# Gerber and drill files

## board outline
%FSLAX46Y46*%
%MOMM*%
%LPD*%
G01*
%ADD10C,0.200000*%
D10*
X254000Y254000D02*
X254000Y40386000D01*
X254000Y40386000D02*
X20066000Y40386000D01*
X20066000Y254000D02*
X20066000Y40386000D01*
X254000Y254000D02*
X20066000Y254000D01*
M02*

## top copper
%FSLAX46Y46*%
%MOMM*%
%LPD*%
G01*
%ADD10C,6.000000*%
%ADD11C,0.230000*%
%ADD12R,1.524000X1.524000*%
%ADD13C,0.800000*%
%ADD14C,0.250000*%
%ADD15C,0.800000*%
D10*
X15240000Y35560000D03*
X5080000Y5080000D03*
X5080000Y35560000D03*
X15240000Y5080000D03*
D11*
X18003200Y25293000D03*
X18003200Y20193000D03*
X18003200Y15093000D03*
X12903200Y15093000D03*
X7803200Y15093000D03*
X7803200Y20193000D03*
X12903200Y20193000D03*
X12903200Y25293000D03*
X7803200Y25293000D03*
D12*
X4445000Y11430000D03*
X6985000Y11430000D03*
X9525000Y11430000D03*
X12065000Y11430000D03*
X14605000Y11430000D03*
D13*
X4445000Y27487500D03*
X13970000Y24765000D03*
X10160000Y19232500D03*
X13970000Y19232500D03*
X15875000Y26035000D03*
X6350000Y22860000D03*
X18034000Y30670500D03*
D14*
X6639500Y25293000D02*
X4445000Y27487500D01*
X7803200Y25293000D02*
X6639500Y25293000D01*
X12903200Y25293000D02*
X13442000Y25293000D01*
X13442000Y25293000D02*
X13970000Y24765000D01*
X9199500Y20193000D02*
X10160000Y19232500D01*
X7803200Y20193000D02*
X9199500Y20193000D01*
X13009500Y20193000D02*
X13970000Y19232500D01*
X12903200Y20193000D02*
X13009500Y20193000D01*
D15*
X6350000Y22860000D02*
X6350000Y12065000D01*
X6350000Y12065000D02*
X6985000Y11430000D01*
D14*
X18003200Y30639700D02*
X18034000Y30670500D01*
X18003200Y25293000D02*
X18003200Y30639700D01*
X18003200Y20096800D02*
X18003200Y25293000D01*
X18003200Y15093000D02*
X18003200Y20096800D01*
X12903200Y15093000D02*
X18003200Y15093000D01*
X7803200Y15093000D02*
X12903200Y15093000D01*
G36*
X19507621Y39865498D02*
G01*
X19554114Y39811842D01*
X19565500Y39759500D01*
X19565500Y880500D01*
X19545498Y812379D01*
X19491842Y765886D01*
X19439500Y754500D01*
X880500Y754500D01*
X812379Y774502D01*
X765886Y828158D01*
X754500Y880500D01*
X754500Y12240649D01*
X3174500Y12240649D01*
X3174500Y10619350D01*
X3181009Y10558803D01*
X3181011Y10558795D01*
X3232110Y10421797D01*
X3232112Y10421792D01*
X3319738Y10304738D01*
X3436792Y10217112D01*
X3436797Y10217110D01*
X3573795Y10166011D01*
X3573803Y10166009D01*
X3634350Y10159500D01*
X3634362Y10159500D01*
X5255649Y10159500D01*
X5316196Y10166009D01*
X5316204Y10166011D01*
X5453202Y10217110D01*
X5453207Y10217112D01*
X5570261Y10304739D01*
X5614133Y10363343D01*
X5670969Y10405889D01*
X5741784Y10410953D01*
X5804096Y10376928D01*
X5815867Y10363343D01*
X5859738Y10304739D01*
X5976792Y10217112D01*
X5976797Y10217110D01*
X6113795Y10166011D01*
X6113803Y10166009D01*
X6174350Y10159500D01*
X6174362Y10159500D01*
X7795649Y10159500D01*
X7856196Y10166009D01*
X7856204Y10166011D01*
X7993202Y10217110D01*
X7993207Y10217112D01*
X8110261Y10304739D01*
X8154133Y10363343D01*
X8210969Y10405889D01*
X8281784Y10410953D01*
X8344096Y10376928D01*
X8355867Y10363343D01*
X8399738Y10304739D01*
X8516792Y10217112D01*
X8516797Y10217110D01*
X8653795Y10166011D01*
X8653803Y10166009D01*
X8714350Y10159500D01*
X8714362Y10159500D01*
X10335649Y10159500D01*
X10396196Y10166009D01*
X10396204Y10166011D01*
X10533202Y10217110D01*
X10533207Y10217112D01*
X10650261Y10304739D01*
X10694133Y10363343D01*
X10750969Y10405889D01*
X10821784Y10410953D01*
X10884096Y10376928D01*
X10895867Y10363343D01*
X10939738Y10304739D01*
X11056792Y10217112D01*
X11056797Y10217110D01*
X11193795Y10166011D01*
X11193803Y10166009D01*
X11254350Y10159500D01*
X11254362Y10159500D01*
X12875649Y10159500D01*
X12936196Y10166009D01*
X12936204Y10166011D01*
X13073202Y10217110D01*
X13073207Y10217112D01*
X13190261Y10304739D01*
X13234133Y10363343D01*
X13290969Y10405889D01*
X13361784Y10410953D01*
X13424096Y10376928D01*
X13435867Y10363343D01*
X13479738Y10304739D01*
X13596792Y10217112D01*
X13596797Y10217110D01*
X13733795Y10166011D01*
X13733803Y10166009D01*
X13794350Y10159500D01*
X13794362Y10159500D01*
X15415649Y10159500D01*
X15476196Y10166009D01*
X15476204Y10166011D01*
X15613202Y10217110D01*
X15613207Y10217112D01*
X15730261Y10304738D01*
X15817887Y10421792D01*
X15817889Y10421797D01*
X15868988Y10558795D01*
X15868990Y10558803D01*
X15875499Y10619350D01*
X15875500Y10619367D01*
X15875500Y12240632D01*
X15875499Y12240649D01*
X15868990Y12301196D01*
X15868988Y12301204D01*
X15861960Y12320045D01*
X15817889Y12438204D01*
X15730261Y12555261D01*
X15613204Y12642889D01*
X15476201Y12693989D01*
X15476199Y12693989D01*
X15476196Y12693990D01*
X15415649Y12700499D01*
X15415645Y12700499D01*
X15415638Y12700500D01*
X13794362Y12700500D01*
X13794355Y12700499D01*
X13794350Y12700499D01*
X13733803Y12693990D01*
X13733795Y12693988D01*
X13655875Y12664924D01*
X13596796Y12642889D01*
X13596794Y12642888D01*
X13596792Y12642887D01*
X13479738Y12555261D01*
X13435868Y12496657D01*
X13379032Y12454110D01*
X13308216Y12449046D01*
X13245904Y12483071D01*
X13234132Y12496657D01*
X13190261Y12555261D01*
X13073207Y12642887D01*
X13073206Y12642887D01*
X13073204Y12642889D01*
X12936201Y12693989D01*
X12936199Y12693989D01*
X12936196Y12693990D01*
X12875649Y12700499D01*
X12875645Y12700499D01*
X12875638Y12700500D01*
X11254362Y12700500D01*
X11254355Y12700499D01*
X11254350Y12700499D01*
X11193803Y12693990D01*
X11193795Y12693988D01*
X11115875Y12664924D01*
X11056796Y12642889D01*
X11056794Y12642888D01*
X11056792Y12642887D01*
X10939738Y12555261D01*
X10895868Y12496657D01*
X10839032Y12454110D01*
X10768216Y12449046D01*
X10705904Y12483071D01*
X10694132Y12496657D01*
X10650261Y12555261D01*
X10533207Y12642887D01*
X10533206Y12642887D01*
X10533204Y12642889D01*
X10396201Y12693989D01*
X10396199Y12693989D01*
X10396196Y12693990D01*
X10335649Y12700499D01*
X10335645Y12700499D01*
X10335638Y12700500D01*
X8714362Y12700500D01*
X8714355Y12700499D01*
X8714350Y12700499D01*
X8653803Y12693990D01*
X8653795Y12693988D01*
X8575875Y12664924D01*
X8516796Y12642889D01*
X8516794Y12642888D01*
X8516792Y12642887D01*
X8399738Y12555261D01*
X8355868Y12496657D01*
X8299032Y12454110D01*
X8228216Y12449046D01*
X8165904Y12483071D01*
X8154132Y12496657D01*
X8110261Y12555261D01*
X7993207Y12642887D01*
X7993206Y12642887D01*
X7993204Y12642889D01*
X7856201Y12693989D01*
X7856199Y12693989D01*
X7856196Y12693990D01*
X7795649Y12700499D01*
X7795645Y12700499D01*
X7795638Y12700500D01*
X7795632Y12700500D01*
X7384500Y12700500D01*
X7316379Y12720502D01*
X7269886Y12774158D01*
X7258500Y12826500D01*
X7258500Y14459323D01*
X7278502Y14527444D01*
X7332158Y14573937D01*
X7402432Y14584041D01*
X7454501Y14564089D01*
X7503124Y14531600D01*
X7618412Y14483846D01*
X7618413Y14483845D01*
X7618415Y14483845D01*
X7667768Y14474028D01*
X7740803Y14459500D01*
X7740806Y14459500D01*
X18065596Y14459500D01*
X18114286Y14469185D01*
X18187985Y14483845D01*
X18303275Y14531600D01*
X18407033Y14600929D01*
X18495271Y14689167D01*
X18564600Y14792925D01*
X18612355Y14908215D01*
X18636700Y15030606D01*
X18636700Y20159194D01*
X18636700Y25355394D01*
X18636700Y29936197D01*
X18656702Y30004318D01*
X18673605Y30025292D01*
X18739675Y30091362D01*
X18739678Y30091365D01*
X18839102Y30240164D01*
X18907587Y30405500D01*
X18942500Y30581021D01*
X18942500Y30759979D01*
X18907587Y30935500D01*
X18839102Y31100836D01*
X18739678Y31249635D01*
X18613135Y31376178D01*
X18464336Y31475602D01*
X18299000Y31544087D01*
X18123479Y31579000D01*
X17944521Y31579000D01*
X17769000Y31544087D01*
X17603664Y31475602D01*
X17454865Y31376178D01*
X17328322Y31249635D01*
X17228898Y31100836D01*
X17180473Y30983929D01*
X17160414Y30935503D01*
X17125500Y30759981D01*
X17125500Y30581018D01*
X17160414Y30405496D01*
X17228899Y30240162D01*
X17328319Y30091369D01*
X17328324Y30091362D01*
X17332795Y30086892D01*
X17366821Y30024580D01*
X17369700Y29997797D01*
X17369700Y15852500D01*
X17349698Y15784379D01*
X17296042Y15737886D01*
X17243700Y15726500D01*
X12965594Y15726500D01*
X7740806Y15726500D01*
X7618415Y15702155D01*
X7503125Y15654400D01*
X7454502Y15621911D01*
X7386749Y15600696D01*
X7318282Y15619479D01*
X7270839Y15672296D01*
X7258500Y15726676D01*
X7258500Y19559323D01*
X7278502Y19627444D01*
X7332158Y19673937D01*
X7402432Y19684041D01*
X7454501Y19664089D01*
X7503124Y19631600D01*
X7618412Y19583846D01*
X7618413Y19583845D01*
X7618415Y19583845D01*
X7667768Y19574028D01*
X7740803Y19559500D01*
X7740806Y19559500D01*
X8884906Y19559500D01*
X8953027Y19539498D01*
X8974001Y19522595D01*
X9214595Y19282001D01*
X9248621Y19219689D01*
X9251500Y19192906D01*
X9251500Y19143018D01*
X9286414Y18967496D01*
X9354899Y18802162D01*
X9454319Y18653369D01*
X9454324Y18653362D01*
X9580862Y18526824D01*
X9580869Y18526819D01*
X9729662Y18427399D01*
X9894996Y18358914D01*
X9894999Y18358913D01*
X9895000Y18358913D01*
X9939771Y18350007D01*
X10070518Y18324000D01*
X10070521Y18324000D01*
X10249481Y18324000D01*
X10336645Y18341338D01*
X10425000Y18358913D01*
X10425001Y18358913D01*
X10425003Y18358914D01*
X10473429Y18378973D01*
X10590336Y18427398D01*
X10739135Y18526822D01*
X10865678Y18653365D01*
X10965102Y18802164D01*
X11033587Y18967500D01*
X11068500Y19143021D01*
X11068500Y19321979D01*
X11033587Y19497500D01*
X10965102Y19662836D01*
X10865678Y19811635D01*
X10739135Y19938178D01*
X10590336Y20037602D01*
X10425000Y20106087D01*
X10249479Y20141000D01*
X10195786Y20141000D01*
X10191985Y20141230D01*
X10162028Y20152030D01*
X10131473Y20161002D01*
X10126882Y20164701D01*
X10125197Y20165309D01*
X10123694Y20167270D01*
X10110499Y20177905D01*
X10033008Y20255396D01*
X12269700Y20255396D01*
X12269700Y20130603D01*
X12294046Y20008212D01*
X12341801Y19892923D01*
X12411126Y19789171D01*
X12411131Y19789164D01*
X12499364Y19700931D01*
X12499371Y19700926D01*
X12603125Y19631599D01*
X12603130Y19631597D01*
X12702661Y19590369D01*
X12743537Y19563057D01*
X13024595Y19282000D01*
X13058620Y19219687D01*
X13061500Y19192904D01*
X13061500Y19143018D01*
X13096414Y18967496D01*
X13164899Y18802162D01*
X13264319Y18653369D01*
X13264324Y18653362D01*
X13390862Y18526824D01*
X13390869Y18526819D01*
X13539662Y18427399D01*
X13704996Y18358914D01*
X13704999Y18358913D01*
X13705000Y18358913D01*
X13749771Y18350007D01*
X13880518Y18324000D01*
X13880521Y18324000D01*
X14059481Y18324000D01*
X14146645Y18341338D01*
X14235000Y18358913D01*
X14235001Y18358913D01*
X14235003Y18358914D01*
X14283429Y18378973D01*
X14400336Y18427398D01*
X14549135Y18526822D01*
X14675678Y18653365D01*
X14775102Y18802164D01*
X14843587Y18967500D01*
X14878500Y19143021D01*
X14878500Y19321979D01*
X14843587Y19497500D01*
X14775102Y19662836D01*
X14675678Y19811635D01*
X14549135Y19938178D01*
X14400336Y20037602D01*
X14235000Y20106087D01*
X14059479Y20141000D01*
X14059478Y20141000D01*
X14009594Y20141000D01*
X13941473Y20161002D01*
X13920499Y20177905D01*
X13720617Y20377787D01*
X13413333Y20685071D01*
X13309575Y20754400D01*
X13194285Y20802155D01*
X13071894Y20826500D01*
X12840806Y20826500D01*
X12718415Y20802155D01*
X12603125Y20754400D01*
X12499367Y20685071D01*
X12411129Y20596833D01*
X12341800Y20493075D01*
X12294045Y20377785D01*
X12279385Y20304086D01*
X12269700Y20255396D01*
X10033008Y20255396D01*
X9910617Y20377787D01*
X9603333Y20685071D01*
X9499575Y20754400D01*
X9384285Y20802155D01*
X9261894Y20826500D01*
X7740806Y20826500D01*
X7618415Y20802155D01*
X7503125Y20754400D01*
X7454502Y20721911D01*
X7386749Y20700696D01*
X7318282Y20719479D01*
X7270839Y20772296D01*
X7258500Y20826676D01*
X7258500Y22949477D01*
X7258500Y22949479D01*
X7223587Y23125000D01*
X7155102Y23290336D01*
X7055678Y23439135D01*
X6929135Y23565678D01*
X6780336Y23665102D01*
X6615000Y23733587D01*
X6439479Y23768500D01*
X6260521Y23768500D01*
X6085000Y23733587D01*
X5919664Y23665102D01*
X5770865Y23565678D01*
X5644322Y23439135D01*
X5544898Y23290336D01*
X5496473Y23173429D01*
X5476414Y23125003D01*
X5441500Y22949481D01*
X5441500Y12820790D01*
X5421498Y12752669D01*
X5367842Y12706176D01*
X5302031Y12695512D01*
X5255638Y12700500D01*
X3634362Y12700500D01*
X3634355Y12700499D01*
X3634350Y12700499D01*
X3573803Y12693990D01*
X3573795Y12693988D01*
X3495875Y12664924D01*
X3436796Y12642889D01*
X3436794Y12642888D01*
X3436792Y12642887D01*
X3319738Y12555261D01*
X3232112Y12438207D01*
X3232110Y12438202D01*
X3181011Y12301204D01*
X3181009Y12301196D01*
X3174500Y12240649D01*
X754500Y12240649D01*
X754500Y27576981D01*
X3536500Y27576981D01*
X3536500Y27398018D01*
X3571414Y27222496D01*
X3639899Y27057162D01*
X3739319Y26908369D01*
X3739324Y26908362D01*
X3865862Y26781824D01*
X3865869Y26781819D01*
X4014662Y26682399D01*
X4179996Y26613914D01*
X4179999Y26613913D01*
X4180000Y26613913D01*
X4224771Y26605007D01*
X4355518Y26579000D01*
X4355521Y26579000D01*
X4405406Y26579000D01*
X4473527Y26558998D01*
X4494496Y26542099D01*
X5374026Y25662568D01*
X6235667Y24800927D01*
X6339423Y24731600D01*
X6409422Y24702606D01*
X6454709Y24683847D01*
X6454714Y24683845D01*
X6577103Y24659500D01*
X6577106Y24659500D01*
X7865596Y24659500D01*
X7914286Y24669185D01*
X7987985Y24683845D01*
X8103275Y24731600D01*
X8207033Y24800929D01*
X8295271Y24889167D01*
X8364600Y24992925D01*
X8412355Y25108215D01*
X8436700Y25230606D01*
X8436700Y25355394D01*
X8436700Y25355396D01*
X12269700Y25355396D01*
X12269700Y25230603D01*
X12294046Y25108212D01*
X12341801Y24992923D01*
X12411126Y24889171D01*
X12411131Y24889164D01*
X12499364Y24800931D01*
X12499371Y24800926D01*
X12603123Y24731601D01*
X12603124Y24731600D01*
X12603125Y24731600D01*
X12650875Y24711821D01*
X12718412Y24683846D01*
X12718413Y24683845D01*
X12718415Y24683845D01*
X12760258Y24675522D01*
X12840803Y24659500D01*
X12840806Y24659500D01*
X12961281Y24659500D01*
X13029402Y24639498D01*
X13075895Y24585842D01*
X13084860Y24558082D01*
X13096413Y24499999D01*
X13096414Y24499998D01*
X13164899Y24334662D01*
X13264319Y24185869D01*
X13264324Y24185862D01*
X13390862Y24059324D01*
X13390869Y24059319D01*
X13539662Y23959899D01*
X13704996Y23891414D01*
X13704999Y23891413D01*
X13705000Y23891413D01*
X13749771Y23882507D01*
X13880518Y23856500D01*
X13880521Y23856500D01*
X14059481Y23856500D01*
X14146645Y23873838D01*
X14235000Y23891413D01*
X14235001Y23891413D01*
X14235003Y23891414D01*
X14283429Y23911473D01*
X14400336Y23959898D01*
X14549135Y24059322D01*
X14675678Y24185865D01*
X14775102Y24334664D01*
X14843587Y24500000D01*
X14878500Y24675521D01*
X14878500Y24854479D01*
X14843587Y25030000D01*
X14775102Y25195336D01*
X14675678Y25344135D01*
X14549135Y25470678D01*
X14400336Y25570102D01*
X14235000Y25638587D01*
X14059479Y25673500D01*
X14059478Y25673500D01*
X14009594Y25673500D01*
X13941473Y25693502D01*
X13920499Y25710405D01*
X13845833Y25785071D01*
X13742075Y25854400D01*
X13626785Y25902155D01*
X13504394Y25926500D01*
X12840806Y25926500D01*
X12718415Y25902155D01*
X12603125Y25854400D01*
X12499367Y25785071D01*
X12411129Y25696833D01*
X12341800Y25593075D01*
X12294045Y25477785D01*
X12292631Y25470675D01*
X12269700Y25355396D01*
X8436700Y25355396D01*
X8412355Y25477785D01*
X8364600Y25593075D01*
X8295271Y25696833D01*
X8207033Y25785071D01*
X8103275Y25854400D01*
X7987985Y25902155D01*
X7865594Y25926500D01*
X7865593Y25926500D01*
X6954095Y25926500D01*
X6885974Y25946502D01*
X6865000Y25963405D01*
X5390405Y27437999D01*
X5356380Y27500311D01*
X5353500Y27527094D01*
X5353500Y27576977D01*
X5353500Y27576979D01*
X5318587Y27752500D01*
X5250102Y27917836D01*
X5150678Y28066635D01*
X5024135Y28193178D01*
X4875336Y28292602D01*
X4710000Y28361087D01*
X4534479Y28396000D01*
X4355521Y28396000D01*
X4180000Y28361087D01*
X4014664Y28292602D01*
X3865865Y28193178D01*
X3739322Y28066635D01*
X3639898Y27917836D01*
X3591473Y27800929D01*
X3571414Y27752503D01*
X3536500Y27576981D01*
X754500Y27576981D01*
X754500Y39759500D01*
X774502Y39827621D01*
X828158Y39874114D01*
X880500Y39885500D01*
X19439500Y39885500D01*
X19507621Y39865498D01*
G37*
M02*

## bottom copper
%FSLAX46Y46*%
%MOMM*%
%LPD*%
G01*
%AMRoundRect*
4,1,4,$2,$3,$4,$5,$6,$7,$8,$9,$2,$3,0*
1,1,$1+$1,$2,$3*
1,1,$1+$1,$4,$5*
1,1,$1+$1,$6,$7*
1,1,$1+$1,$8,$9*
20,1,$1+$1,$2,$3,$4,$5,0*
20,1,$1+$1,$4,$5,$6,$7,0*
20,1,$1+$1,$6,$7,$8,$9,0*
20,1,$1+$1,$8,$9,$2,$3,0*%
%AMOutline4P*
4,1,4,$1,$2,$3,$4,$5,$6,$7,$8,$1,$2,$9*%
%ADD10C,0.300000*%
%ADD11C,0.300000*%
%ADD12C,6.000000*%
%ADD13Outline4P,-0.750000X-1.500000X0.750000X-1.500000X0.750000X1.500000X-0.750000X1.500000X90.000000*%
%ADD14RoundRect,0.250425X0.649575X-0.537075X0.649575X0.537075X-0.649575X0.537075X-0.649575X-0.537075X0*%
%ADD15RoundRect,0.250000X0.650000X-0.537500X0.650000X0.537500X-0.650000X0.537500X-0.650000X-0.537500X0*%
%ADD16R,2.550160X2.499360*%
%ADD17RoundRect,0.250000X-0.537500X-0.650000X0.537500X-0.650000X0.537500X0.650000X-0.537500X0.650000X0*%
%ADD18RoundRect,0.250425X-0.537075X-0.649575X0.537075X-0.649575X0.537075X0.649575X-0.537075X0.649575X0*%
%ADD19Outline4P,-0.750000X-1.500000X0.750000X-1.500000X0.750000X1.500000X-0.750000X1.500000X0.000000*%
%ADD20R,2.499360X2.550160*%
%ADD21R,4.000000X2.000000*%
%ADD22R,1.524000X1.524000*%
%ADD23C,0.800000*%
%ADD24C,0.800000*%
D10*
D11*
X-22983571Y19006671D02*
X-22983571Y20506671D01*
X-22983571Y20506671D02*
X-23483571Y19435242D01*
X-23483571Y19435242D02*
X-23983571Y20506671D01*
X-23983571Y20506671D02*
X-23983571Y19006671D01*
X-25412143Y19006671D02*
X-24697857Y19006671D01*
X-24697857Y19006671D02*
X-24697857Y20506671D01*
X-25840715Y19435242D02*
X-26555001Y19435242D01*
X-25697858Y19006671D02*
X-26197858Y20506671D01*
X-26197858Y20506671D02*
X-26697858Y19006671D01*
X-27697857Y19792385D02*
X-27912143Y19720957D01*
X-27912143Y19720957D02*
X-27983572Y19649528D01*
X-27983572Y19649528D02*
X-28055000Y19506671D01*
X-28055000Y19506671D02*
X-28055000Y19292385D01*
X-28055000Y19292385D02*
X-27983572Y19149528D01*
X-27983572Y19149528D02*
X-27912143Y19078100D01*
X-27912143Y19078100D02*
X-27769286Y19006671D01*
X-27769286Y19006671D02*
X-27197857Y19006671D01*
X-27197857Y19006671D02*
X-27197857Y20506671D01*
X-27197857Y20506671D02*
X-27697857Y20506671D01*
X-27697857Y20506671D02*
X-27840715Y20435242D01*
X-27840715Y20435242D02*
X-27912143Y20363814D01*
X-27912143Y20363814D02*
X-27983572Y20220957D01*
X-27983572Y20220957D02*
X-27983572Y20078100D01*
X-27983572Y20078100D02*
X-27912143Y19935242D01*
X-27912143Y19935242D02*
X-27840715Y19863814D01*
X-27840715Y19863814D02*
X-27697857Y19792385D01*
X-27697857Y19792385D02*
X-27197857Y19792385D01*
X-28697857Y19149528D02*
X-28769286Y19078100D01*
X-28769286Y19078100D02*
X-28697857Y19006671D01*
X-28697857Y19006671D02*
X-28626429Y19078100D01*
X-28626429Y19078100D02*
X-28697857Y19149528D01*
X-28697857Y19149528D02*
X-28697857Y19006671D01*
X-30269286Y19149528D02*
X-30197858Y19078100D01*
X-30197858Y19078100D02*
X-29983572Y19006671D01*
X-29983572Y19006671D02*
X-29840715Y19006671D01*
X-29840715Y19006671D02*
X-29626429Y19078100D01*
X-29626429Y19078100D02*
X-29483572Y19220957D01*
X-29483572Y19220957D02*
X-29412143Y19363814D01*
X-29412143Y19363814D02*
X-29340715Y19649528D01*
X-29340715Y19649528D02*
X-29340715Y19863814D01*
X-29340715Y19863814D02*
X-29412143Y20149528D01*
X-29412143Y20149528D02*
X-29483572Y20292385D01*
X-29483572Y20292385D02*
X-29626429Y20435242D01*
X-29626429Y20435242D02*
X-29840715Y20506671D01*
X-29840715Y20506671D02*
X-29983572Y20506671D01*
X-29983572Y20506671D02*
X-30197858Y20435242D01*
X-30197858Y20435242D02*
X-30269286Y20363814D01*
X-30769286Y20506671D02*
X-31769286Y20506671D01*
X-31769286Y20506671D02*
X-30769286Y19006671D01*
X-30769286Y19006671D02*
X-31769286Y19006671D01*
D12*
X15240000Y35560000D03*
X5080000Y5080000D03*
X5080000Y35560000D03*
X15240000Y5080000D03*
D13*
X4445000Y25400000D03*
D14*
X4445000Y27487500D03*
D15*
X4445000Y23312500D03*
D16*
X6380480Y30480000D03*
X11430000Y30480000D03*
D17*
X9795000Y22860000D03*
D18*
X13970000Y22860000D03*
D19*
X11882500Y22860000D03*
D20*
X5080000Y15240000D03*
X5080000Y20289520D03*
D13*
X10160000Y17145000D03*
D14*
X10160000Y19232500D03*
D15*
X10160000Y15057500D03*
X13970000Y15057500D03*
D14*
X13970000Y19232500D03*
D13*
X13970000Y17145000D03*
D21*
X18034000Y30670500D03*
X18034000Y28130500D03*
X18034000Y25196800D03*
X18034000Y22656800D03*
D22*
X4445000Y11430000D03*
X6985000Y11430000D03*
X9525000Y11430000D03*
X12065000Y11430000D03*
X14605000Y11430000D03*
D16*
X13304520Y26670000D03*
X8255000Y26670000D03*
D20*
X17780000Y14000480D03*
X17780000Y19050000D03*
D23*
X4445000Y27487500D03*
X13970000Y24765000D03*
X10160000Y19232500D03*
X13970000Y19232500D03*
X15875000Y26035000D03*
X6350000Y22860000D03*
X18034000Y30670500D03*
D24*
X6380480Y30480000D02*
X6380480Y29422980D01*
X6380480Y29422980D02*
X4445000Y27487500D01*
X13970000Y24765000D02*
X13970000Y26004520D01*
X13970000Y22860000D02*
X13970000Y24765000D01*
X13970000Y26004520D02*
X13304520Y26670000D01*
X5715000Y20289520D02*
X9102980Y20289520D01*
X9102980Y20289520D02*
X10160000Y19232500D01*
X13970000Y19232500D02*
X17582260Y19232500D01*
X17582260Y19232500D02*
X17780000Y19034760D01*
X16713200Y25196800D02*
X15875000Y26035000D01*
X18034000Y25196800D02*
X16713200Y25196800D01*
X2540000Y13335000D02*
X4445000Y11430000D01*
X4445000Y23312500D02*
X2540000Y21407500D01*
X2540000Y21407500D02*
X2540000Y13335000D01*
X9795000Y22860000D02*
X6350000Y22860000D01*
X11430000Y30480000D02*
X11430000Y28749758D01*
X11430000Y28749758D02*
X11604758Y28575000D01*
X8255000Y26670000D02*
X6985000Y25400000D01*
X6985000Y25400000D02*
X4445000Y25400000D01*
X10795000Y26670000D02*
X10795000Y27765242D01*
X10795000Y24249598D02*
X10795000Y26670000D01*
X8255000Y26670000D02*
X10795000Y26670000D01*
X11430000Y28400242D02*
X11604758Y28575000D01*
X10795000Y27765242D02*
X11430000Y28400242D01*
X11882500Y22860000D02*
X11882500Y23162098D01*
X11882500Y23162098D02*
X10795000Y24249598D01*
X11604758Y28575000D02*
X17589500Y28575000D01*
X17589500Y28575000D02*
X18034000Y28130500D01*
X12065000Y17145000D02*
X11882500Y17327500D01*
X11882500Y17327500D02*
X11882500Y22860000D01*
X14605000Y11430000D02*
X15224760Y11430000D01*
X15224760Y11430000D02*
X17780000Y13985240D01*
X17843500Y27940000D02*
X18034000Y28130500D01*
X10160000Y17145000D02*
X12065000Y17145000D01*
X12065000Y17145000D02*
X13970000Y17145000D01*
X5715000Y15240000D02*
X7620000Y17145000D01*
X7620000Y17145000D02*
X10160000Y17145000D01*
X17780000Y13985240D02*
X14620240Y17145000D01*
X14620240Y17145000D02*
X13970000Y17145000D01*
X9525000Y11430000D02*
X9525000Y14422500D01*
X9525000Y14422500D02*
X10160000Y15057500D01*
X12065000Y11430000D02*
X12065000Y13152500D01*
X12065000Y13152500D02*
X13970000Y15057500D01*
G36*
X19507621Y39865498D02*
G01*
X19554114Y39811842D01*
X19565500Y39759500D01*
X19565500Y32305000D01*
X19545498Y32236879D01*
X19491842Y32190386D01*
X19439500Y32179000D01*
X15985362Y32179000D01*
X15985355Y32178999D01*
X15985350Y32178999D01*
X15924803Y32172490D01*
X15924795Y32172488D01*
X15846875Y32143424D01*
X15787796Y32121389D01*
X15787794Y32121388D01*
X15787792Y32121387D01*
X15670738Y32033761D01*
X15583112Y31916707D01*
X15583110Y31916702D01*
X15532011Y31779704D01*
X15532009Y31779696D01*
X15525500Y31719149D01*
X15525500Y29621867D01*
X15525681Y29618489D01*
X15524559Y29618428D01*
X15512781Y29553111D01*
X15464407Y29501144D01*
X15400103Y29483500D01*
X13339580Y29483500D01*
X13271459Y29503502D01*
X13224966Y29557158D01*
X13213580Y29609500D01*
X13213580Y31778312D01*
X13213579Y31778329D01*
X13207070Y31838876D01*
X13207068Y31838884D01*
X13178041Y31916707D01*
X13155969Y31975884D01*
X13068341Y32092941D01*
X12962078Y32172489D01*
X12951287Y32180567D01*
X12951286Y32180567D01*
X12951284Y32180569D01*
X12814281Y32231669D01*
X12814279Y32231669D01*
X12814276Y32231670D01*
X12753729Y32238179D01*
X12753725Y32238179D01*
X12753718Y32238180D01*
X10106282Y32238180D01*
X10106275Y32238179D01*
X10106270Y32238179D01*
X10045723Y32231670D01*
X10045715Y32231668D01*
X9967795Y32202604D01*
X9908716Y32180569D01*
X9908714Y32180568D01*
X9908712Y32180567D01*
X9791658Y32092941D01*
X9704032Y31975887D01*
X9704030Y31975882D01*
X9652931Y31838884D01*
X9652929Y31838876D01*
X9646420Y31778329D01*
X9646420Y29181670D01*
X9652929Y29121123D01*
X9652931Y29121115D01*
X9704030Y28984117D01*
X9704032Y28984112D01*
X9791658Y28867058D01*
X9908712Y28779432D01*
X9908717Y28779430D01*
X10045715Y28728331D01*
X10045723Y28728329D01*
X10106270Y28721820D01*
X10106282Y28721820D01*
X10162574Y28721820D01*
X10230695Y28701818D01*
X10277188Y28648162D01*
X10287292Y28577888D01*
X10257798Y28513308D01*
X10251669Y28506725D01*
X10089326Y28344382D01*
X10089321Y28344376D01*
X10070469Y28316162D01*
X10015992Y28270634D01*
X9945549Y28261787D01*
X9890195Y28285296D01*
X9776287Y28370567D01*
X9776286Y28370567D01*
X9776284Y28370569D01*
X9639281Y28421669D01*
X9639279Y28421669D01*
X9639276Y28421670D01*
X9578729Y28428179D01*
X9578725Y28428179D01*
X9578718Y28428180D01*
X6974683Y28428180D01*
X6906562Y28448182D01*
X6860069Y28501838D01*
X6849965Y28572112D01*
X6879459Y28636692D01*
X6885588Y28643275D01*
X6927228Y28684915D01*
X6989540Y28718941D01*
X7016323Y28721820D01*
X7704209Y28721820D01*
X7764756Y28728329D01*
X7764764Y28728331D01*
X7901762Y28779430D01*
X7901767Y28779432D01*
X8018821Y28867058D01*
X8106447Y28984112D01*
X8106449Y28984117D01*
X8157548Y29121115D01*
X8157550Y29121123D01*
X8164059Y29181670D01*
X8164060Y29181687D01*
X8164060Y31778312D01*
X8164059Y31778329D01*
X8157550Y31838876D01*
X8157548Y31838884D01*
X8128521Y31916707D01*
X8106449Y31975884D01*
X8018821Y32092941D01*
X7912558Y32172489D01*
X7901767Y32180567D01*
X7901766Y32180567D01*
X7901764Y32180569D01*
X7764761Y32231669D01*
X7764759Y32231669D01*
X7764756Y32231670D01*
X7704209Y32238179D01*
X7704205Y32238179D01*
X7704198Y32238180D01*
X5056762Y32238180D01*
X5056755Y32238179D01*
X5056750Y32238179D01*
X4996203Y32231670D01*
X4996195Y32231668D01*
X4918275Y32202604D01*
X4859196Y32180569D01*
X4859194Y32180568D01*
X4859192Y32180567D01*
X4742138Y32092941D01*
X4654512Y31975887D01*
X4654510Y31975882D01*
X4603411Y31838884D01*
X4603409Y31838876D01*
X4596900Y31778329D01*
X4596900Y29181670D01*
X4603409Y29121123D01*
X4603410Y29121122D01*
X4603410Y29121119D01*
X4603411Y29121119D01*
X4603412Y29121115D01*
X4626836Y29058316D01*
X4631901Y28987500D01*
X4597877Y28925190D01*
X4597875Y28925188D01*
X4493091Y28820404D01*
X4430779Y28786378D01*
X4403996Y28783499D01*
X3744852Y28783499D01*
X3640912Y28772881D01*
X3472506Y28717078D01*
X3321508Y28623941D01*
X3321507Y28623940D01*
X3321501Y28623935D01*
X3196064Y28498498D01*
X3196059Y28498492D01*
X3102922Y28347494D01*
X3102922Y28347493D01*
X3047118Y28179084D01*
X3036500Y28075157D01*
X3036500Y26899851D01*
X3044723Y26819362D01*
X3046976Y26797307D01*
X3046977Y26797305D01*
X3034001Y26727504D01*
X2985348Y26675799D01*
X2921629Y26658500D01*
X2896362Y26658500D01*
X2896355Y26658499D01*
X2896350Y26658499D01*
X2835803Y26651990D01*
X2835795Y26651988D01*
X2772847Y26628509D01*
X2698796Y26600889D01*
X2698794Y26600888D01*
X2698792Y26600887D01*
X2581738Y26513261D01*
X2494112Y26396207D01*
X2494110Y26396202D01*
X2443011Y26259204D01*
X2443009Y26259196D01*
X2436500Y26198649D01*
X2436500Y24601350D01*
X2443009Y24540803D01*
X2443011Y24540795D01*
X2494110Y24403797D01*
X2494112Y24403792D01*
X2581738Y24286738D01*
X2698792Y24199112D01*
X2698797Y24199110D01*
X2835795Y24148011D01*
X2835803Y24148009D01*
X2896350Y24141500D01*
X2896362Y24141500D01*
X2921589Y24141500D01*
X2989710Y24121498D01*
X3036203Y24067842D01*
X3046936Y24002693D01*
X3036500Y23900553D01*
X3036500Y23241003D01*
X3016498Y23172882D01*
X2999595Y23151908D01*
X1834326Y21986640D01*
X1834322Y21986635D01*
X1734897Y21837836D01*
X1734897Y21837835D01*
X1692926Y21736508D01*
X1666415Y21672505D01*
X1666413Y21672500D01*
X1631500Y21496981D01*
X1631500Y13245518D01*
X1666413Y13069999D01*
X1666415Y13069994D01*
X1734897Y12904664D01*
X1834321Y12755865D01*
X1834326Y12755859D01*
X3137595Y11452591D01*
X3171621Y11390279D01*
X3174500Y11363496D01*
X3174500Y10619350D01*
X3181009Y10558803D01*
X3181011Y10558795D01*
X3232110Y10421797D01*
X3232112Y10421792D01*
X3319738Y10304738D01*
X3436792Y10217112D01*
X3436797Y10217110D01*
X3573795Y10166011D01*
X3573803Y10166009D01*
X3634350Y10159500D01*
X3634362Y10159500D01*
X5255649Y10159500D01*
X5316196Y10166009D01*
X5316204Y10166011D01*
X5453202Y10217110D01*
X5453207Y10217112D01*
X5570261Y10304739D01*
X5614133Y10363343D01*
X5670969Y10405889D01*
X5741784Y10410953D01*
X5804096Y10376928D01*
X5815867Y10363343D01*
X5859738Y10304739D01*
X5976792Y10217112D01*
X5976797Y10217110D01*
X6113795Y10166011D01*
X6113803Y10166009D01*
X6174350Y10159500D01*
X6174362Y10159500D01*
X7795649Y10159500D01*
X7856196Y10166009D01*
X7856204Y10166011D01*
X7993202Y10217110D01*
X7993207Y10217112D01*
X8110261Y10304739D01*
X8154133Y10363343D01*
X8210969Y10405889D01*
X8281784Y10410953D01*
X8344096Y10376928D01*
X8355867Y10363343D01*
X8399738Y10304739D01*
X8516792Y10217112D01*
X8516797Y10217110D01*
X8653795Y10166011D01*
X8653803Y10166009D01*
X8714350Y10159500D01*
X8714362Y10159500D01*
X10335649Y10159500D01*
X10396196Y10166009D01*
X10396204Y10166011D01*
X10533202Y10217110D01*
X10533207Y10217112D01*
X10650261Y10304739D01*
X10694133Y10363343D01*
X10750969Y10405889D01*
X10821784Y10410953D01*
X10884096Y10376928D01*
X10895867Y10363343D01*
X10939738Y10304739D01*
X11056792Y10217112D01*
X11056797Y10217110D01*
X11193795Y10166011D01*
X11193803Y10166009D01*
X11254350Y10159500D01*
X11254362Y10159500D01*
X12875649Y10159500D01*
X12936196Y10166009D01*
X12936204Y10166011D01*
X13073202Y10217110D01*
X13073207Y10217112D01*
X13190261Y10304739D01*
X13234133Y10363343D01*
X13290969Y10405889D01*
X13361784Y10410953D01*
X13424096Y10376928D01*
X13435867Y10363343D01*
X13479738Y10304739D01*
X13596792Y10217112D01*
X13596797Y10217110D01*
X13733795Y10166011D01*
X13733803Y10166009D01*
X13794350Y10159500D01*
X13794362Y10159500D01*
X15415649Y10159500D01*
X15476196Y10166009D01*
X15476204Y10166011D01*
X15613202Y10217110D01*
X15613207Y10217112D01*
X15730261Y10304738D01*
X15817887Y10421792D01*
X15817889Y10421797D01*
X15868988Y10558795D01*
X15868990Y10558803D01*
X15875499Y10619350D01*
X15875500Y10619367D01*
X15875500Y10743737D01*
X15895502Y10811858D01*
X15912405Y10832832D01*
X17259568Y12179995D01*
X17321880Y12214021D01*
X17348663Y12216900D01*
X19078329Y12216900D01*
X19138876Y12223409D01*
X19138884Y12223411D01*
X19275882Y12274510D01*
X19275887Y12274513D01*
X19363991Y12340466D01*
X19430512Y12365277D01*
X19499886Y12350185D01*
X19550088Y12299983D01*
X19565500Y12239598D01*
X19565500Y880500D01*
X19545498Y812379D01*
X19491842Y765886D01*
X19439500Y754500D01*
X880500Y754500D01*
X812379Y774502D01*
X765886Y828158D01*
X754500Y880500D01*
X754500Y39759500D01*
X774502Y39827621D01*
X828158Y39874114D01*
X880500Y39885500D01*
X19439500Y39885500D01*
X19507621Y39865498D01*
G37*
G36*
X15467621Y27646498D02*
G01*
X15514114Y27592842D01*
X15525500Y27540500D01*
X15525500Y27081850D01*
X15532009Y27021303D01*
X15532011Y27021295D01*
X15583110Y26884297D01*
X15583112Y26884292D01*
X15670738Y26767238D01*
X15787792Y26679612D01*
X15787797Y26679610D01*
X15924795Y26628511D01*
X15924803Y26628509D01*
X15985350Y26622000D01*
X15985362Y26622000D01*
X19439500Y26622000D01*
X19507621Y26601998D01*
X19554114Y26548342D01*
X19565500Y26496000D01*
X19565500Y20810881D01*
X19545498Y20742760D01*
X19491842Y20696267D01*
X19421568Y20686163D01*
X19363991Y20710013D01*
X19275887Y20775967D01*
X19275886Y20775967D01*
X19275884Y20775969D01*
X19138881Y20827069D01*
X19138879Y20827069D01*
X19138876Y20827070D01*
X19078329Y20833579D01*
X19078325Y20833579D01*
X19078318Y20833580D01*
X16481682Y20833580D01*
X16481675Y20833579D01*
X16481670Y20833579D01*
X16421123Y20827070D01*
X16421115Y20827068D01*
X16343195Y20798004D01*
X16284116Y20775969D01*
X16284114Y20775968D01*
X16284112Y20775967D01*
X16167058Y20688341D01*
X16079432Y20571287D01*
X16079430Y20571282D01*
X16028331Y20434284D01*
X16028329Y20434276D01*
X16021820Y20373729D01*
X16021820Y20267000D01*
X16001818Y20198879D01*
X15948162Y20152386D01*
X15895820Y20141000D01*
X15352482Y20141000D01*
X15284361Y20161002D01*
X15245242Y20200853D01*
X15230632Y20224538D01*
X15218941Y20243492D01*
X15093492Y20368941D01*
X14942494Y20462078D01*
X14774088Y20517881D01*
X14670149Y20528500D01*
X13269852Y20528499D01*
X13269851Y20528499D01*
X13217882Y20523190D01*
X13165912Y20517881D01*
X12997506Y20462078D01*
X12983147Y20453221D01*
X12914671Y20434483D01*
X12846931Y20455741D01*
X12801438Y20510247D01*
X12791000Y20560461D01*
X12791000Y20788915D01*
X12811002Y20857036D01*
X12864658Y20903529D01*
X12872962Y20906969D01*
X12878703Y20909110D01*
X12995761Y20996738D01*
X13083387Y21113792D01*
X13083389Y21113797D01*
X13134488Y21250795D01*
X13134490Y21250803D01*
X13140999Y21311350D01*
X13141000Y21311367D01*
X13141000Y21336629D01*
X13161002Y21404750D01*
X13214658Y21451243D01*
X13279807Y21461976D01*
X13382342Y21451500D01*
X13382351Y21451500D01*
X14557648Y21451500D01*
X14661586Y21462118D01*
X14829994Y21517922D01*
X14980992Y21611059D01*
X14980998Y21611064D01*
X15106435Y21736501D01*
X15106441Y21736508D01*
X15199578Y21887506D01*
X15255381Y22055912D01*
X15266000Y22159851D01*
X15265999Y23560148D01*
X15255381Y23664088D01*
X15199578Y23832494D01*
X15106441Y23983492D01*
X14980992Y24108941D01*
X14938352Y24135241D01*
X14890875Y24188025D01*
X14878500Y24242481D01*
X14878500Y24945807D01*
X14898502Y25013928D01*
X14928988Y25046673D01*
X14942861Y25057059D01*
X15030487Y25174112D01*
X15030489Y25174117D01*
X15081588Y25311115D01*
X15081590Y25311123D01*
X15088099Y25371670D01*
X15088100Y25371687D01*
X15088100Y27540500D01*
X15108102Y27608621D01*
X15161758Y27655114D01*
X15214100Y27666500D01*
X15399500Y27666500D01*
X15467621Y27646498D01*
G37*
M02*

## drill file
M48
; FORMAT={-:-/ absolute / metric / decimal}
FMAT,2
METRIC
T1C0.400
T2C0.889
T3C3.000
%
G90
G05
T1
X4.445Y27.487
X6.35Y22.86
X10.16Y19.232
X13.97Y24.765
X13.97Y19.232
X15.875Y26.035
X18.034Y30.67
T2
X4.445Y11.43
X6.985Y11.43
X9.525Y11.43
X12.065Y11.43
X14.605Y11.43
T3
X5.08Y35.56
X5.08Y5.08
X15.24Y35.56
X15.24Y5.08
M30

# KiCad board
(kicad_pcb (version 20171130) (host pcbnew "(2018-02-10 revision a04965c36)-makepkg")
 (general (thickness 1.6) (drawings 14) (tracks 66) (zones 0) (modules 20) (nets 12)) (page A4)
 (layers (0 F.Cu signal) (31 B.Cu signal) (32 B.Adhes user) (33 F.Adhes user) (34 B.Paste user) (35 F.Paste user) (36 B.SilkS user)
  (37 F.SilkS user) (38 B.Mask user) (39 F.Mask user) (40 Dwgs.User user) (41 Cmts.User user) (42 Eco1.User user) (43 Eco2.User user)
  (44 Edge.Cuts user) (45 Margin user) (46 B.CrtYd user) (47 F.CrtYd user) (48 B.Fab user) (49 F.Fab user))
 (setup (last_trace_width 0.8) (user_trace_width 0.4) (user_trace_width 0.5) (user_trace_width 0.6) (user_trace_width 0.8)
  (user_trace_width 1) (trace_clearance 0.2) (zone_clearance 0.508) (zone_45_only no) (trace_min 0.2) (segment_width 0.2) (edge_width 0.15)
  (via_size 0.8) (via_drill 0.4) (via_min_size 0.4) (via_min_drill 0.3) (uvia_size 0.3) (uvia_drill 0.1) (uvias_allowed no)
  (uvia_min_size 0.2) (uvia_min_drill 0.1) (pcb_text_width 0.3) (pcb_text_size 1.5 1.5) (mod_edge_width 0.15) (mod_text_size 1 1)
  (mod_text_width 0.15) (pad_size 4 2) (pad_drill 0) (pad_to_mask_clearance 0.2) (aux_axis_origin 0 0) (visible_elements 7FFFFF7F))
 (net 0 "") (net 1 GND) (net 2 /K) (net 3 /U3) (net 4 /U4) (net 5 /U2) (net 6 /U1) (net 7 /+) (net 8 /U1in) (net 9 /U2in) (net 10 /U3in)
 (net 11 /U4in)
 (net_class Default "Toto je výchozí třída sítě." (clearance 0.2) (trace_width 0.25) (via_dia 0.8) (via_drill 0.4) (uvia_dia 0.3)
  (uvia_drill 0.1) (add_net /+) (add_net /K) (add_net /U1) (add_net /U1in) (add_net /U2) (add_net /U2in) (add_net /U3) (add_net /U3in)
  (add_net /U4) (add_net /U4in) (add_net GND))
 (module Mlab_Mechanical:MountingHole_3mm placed (layer F.Cu) (at 15.24 -35.56)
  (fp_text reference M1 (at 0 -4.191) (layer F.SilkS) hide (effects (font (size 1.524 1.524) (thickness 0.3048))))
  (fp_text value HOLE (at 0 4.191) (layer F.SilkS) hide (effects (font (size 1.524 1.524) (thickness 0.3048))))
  (pad 1 thru_hole circle (at 0 0) (size 6 6) (drill 3) (layers *.Cu *.Adhes *.Mask) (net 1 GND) (clearance 1) (zone_connect 2)))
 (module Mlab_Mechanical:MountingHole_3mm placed (layer F.Cu) (at 5.08 -5.08)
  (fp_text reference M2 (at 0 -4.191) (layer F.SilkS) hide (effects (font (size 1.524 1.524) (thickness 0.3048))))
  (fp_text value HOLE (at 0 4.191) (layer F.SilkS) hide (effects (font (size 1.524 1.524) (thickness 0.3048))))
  (pad 1 thru_hole circle (at 0 0) (size 6 6) (drill 3) (layers *.Cu *.Adhes *.Mask) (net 1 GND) (clearance 1) (zone_connect 2)))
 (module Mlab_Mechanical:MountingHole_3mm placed (layer F.Cu) (at 5.08 -35.56)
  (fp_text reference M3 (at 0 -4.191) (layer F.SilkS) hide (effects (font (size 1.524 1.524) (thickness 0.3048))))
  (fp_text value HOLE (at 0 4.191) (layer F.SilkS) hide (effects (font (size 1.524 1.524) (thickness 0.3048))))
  (pad 1 thru_hole circle (at 0 0) (size 6 6) (drill 3) (layers *.Cu *.Adhes *.Mask) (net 1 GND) (clearance 1) (zone_connect 2)))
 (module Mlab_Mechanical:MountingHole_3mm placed (layer F.Cu) (at 15.24 -5.08)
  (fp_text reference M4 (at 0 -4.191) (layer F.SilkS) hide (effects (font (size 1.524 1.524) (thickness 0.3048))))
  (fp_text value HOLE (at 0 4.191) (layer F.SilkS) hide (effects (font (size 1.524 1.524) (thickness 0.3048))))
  (pad 1 thru_hole circle (at 0 0) (size 6 6) (drill 3) (layers *.Cu *.Adhes *.Mask) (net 1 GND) (clearance 1) (zone_connect 2)))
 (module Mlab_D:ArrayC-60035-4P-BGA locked (layer F.Cu) (at 12.9032 -20.193)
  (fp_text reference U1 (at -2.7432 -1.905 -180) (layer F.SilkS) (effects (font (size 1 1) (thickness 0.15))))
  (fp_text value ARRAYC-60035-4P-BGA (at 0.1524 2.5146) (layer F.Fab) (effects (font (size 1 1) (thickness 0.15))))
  (pad A3 smd circle (at 5.1 -5.1) (size 0.23 0.23) (layers F.Cu F.Paste F.Mask) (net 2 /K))
  (pad B3 smd circle (at 5.1 0) (size 0.23 0.23) (layers F.Cu F.Paste F.Mask) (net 2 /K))
  (pad C3 smd circle (at 5.1 5.1) (size 0.23 0.23) (layers F.Cu F.Paste F.Mask) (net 2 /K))
  (pad C2 smd circle (at 0 5.1) (size 0.23 0.23) (layers F.Cu F.Paste F.Mask) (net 2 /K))
  (pad C1 smd circle (at -5.1 5.1) (size 0.23 0.23) (layers F.Cu F.Paste F.Mask) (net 2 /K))
  (pad B1 smd circle (at -5.1 0) (size 0.23 0.23) (layers F.Cu F.Paste F.Mask) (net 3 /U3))
  (pad B2 smd circle (at 0 0) (size 0.23 0.23) (layers F.Cu F.Paste F.Mask) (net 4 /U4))
  (pad A2 smd circle (at 0 -5.1) (size 0.23 0.23) (layers F.Cu F.Paste F.Mask) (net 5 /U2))
  (pad A1 smd circle (at -5.1 -5.1) (size 0.23 0.23) (layers F.Cu F.Paste F.Mask) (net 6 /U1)))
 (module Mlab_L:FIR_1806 (layer B.Cu) (at 4.445 -25.4 90)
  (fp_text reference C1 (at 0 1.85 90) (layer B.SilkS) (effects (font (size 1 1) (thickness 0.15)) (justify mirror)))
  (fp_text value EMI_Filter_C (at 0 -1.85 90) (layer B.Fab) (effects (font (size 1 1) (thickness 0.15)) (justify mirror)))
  (pad 2 smd trapezoid (at 0 0 90) (size 1.5 3) (layers B.Cu B.Paste B.Mask) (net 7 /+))
  (pad 3 smd roundrect (at 2.0875 0 90) (size 1.575 1.8) (layers B.Cu B.Paste B.Mask) (roundrect_rratio 0.159) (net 6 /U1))
  (pad 1 smd roundrect (at -2.0875 0 90) (size 1.575 1.8) (layers B.Cu B.Paste B.Mask) (roundrect_rratio 0.15873) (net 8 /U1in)))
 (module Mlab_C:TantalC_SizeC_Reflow (layer B.Cu) (at 8.90524 -30.48 180)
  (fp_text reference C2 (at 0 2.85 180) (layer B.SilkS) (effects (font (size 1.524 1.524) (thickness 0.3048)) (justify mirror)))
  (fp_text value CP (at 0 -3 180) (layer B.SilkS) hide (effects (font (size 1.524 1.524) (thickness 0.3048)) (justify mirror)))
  (pad 2 smd rect (at 2.52476 0 180) (size 2.55016 2.49936) (layers B.Cu B.Paste B.Mask) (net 6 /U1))
  (pad 1 smd rect (at -2.52476 0 180) (size 2.55016 2.49936) (layers B.Cu B.Paste B.Mask) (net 7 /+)))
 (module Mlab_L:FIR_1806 (layer B.Cu) (at 11.8825 -22.86)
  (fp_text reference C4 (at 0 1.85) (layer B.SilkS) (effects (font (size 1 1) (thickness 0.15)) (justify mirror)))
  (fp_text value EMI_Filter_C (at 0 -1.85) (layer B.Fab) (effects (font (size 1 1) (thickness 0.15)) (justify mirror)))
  (pad 1 smd roundrect (at -2.0875 0) (size 1.575 1.8) (layers B.Cu B.Paste B.Mask) (roundrect_rratio 0.15873) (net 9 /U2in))
  (pad 3 smd roundrect (at 2.0875 0) (size 1.575 1.8) (layers B.Cu B.Paste B.Mask) (roundrect_rratio 0.159) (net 5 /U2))
  (pad 2 smd trapezoid (at 0 0) (size 1.5 3) (layers B.Cu B.Paste B.Mask) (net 7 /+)))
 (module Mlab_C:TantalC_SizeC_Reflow (layer B.Cu) (at 5.08 -17.76476 90)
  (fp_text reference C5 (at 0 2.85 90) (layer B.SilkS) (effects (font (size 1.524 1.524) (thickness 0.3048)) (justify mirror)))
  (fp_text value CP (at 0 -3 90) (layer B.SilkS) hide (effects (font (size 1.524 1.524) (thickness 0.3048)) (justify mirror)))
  (pad 1 smd rect (at -2.52476 0 90) (size 2.55016 2.49936) (layers B.Cu B.Paste B.Mask) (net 7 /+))
  (pad 2 smd rect (at 2.52476 0 90) (size 2.55016 2.49936) (layers B.Cu B.Paste B.Mask) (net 3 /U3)))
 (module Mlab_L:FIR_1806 (layer B.Cu) (at 10.16 -17.145 90)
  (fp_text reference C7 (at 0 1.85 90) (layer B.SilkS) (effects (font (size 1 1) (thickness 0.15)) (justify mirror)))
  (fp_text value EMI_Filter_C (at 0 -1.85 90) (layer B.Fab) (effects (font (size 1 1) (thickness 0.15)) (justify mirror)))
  (pad 2 smd trapezoid (at 0 0 90) (size 1.5 3) (layers B.Cu B.Paste B.Mask) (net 7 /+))
  (pad 3 smd roundrect (at 2.0875 0 90) (size 1.575 1.8) (layers B.Cu B.Paste B.Mask) (roundrect_rratio 0.159) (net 3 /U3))
  (pad 1 smd roundrect (at -2.0875 0 90) (size 1.575 1.8) (layers B.Cu B.Paste B.Mask) (roundrect_rratio 0.15873) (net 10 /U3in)))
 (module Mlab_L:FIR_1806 (layer B.Cu) (at 13.97 -17.145 90)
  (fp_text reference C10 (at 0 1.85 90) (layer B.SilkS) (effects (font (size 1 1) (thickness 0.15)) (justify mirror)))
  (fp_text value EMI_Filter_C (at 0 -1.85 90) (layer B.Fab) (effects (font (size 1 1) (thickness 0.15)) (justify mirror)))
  (pad 1 smd roundrect (at -2.0875 0 90) (size 1.575 1.8) (layers B.Cu B.Paste B.Mask) (roundrect_rratio 0.15873) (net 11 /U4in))
  (pad 3 smd roundrect (at 2.0875 0 90) (size 1.575 1.8) (layers B.Cu B.Paste B.Mask) (roundrect_rratio 0.159) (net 4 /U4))
  (pad 2 smd trapezoid (at 0 0 90) (size 1.5 3) (layers B.Cu B.Paste B.Mask) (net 7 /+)))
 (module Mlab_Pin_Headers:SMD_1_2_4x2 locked (layer B.Cu) (at 18.034 -30.6705 180)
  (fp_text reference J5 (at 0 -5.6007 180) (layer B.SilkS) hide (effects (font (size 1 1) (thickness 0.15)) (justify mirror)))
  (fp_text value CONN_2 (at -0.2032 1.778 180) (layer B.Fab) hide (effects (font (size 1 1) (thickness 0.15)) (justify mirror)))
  (pad 1 smd rect (at 0 0 180) (size 4 2) (layers B.Cu B.Paste B.Mask) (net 2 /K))
  (pad 2 smd rect (at 0 -2.54 180) (size 4 2) (layers B.Cu B.Paste B.Mask) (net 7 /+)))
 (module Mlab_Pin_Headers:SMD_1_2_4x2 (layer B.Cu) (at 18.034 -22.6568)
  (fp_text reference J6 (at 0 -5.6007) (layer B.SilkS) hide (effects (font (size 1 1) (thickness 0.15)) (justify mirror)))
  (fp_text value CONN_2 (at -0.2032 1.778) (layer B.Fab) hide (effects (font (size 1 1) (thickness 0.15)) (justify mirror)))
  (pad 2 smd rect (at 0 -2.54) (size 4 2) (layers B.Cu B.Paste B.Mask) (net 1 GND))
  (pad 1 smd rect (at 0 0) (size 4 2) (layers B.Cu B.Paste B.Mask) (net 1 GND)))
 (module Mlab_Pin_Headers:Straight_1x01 (layer F.Cu) (at 4.445 -11.43 180)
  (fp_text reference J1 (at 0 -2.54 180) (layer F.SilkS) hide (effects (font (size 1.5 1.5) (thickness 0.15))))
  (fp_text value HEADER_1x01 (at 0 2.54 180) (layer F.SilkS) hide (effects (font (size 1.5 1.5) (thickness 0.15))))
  (pad 1 thru_hole rect (at 0 0 180) (size 1.524 1.524) (drill 0.889) (layers *.Cu *.Mask F.SilkS) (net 8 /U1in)))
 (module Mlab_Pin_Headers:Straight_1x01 (layer F.Cu) (at 6.985 -11.43 90)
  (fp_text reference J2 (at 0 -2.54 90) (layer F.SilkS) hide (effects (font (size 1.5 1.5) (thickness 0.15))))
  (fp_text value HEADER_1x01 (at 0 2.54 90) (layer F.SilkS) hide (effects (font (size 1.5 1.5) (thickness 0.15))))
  (pad 1 thru_hole rect (at 0 0 90) (size 1.524 1.524) (drill 0.889) (layers *.Cu *.Mask F.SilkS) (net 9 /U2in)))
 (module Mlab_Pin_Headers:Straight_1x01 (layer F.Cu) (at 9.525 -11.43 90)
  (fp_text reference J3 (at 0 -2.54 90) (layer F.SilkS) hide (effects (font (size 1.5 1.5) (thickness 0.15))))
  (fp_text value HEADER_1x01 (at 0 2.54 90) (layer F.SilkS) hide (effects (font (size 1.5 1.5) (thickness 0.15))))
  (pad 1 thru_hole rect (at 0 0 90) (size 1.524 1.524) (drill 0.889) (layers *.Cu *.Mask F.SilkS) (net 10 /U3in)))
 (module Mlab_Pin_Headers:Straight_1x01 (layer F.Cu) (at 12.065 -11.43 180)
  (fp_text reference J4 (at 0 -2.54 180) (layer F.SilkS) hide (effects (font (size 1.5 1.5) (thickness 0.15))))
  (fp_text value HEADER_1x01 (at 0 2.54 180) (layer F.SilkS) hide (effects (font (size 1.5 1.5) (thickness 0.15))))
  (pad 1 thru_hole rect (at 0 0 180) (size 1.524 1.524) (drill 0.889) (layers *.Cu *.Mask F.SilkS) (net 11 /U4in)))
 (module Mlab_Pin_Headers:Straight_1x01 (layer F.Cu) (at 14.605 -11.43)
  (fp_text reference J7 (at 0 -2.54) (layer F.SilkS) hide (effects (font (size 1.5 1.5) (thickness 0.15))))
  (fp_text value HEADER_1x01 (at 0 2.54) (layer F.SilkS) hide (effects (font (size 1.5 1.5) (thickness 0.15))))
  (pad 1 thru_hole rect (at 0 0) (size 1.524 1.524) (drill 0.889) (layers *.Cu *.Mask F.SilkS) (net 7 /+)))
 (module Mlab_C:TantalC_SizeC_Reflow (layer B.Cu) (at 10.77976 -26.67)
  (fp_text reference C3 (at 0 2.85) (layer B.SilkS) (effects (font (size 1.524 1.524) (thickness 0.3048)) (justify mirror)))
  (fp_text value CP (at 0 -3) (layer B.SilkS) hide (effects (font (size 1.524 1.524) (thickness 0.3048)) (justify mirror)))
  (pad 2 smd rect (at 2.52476 0) (size 2.55016 2.49936) (layers B.Cu B.Paste B.Mask) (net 5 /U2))
  (pad 1 smd rect (at -2.52476 0) (size 2.55016 2.49936) (layers B.Cu B.Paste B.Mask) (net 7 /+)))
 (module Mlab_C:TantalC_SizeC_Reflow (layer B.Cu) (at 17.78 -16.52524 90)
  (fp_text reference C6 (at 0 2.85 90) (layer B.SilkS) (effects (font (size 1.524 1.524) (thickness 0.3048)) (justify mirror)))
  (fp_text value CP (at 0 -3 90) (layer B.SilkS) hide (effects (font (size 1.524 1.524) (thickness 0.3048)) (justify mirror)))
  (pad 1 smd rect (at -2.52476 0 90) (size 2.55016 2.49936) (layers B.Cu B.Paste B.Mask) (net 7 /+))
  (pad 2 smd rect (at 2.52476 0 90) (size 2.55016 2.49936) (layers B.Cu B.Paste B.Mask) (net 4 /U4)))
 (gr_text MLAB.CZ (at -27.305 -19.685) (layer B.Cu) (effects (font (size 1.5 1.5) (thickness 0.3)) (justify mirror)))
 (gr_line (start 0.254 -0.254) (end 0.254 -40.386) (layer Edge.Cuts) (width 0.2))
 (gr_line (start 0.254 -40.386) (end 20.066 -40.386) (layer Edge.Cuts) (width 0.2))
 (gr_line (start 20.066 -0.254) (end 20.066 -40.386) (layer Edge.Cuts) (width 0.2))
 (gr_line (start 0.254 -0.254) (end 20.066 -0.254) (layer Edge.Cuts) (width 0.2))
 (segment (start 6.6395 -25.293) (end 4.445 -27.4875) (width 0.25) (layer F.Cu) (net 6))
 (segment (start 7.8032 -25.293) (end 6.6395 -25.293) (width 0.25) (layer F.Cu) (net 6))
 (via (at 4.445 -27.4875) (size 0.8) (drill 0.4) (layers F.Cu B.Cu) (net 6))
 (segment (start 6.38048 -30.48) (end 6.38048 -29.42298) (width 0.8) (layer B.Cu) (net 6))
 (segment (start 6.38048 -29.42298) (end 4.445 -27.4875) (width 0.8) (layer B.Cu) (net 6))
 (segment (start 13.97 -24.765) (end 13.97 -26.00452) (width 0.8) (layer B.Cu) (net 5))
 (segment (start 13.97 -22.86) (end 13.97 -24.765) (width 0.8) (layer B.Cu) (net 5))
 (segment (start 12.9032 -25.293) (end 13.442 -25.293) (width 0.25) (layer F.Cu) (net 5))
 (segment (start 13.442 -25.293) (end 13.97 -24.765) (width 0.25) (layer F.Cu) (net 5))
 (via (at 13.97 -24.765) (size 0.8) (drill 0.4) (layers F.Cu B.Cu) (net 5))
 (segment (start 13.97 -26.00452) (end 13.30452 -26.67) (width 0.8) (layer B.Cu) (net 5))
 (segment (start 5.715 -20.28952) (end 9.10298 -20.28952) (width 0.8) (layer B.Cu) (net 3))
 (segment (start 9.10298 -20.28952) (end 10.16 -19.2325) (width 0.8) (layer B.Cu) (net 3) (status 20))
 (segment (start 9.1995 -20.193) (end 10.16 -19.2325) (width 0.25) (layer F.Cu) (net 3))
 (segment (start 7.8032 -20.193) (end 9.1995 -20.193) (width 0.25) (layer F.Cu) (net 3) (status 10))
 (via (at 10.16 -19.2325) (size 0.8) (drill 0.4) (layers F.Cu B.Cu) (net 3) (status 30))
 (segment (start 13.97 -19.2325) (end 17.58226 -19.2325) (width 0.8) (layer B.Cu) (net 4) (status 10))
 (segment (start 17.58226 -19.2325) (end 17.78 -19.03476) (width 0.8) (layer B.Cu) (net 4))
 (segment (start 13.0095 -20.193) (end 13.97 -19.2325) (width 0.25) (layer F.Cu) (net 4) (status 10))
 (segment (start 12.9032 -20.193) (end 13.0095 -20.193) (width 0.25) (layer F.Cu) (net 4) (status 30))
 (via (at 13.97 -19.2325) (size 0.8) (drill 0.4) (layers F.Cu B.Cu) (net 4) (status 30))
 (segment (start 16.7132 -25.1968) (end 15.875 -26.035) (width 0.8) (layer B.Cu) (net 1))
 (segment (start 18.034 -25.1968) (end 16.7132 -25.1968) (width 0.8) (layer B.Cu) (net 1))
 (via (at 15.875 -26.035) (size 0.8) (drill 0.4) (layers F.Cu B.Cu) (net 1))
 (segment (start 2.54 -13.335) (end 4.445 -11.43) (width 0.8) (layer B.Cu) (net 8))
 (segment (start 4.445 -23.3125) (end 2.54 -21.4075) (width 0.8) (layer B.Cu) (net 8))
 (segment (start 2.54 -21.4075) (end 2.54 -13.335) (width 0.8) (layer B.Cu) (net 8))
 (segment (start 6.35 -22.86) (end 6.35 -12.065) (width 0.8) (layer F.Cu) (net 9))
 (segment (start 6.35 -12.065) (end 6.985 -11.43) (width 0.8) (layer F.Cu) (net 9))
 (segment (start 9.795 -22.86) (end 6.35 -22.86) (width 0.8) (layer B.Cu) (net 9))
 (via (at 6.35 -22.86) (size 0.8) (drill 0.4) (layers F.Cu B.Cu) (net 9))
 (segment (start 18.0032 -30.6397) (end 18.034 -30.6705) (width 0.25) (layer F.Cu) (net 2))
 (segment (start 18.0032 -25.293) (end 18.0032 -30.6397) (width 0.25) (layer F.Cu) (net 2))
 (via (at 18.034 -30.6705) (size 0.8) (drill 0.4) (layers F.Cu B.Cu) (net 2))
 (segment (start 18.0032 -20.0968) (end 18.0032 -25.293) (width 0.25) (layer F.Cu) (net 2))
 (segment (start 18.0032 -15.093) (end 18.0032 -20.0968) (width 0.25) (layer F.Cu) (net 2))
 (segment (start 12.9032 -15.093) (end 18.0032 -15.093) (width 0.25) (layer F.Cu) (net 2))
 (segment (start 7.8032 -15.093) (end 12.9032 -15.093) (width 0.25) (layer F.Cu) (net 2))
 (segment (start 11.43 -30.48) (end 11.43 -28.749758) (width 0.8) (layer B.Cu) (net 7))
 (segment (start 11.43 -28.749758) (end 11.604758 -28.575) (width 0.8) (layer B.Cu) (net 7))
 (segment (start 8.255 -26.67) (end 6.985 -25.4) (width 0.8) (layer B.Cu) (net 7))
 (segment (start 6.985 -25.4) (end 4.445 -25.4) (width 0.8) (layer B.Cu) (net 7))
 (segment (start 10.795 -26.67) (end 10.795 -27.765242) (width 0.8) (layer B.Cu) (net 7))
 (segment (start 10.795 -24.249598) (end 10.795 -26.67) (width 0.8) (layer B.Cu) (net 7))
 (segment (start 8.255 -26.67) (end 10.795 -26.67) (width 0.8) (layer B.Cu) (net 7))
 (segment (start 11.43 -28.400242) (end 11.604758 -28.575) (width 0.8) (layer B.Cu) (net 7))
 (segment (start 10.795 -27.765242) (end 11.43 -28.400242) (width 0.8) (layer B.Cu) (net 7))
 (segment (start 11.8825 -22.86) (end 11.8825 -23.162098) (width 0.8) (layer B.Cu) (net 7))
 (segment (start 11.8825 -23.162098) (end 10.795 -24.249598) (width 0.8) (layer B.Cu) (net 7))
 (segment (start 11.604758 -28.575) (end 17.5895 -28.575) (width 0.8) (layer B.Cu) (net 7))
 (segment (start 17.5895 -28.575) (end 18.034 -28.1305) (width 0.8) (layer B.Cu) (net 7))
 (segment (start 12.065 -17.145) (end 11.8825 -17.3275) (width 0.8) (layer B.Cu) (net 7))
 (segment (start 11.8825 -17.3275) (end 11.8825 -22.86) (width 0.8) (layer B.Cu) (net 7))
 (segment (start 14.605 -11.43) (end 15.22476 -11.43) (width 0.8) (layer B.Cu) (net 7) (status 30))
 (segment (start 15.22476 -11.43) (end 17.78 -13.98524) (width 0.8) (layer B.Cu) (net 7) (status 10))
 (segment (start 17.8435 -27.94) (end 18.034 -28.1305) (width 0.8) (layer B.Cu) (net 7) (status 30))
 (segment (start 10.16 -17.145) (end 12.065 -17.145) (width 0.8) (layer B.Cu) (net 7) (status 10))
 (segment (start 12.065 -17.145) (end 13.97 -17.145) (width 0.8) (layer B.Cu) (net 7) (status 20))
 (segment (start 5.715 -15.24) (end 7.62 -17.145) (width 0.8) (layer B.Cu) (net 7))
 (segment (start 7.62 -17.145) (end 10.16 -17.145) (width 0.8) (layer B.Cu) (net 7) (status 20))
 (segment (start 17.78 -13.98524) (end 14.62024 -17.145) (width 0.8) (layer B.Cu) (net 7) (status 20))
 (segment (start 14.62024 -17.145) (end 13.97 -17.145) (width 0.8) (layer B.Cu) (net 7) (status 30))
 (segment (start 9.525 -11.43) (end 9.525 -14.4225) (width 0.8) (layer B.Cu) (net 10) (status 30))
 (segment (start 9.525 -14.4225) (end 10.16 -15.0575) (width 0.8) (layer B.Cu) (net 10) (status 30))
 (segment (start 12.065 -11.43) (end 12.065 -13.1525) (width 0.8) (layer B.Cu) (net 11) (status 10))
 (segment (start 12.065 -13.1525) (end 13.97 -15.0575) (width 0.8) (layer B.Cu) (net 11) (status 20))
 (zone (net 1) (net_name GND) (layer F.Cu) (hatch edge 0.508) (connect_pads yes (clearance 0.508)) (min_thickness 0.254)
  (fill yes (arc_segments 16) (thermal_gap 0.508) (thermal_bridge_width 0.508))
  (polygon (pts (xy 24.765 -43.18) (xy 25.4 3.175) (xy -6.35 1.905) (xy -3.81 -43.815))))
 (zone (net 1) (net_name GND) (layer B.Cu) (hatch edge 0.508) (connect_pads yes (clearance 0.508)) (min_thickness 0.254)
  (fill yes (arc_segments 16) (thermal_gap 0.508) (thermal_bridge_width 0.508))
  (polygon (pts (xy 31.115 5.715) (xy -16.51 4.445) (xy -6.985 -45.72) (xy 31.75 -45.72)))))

